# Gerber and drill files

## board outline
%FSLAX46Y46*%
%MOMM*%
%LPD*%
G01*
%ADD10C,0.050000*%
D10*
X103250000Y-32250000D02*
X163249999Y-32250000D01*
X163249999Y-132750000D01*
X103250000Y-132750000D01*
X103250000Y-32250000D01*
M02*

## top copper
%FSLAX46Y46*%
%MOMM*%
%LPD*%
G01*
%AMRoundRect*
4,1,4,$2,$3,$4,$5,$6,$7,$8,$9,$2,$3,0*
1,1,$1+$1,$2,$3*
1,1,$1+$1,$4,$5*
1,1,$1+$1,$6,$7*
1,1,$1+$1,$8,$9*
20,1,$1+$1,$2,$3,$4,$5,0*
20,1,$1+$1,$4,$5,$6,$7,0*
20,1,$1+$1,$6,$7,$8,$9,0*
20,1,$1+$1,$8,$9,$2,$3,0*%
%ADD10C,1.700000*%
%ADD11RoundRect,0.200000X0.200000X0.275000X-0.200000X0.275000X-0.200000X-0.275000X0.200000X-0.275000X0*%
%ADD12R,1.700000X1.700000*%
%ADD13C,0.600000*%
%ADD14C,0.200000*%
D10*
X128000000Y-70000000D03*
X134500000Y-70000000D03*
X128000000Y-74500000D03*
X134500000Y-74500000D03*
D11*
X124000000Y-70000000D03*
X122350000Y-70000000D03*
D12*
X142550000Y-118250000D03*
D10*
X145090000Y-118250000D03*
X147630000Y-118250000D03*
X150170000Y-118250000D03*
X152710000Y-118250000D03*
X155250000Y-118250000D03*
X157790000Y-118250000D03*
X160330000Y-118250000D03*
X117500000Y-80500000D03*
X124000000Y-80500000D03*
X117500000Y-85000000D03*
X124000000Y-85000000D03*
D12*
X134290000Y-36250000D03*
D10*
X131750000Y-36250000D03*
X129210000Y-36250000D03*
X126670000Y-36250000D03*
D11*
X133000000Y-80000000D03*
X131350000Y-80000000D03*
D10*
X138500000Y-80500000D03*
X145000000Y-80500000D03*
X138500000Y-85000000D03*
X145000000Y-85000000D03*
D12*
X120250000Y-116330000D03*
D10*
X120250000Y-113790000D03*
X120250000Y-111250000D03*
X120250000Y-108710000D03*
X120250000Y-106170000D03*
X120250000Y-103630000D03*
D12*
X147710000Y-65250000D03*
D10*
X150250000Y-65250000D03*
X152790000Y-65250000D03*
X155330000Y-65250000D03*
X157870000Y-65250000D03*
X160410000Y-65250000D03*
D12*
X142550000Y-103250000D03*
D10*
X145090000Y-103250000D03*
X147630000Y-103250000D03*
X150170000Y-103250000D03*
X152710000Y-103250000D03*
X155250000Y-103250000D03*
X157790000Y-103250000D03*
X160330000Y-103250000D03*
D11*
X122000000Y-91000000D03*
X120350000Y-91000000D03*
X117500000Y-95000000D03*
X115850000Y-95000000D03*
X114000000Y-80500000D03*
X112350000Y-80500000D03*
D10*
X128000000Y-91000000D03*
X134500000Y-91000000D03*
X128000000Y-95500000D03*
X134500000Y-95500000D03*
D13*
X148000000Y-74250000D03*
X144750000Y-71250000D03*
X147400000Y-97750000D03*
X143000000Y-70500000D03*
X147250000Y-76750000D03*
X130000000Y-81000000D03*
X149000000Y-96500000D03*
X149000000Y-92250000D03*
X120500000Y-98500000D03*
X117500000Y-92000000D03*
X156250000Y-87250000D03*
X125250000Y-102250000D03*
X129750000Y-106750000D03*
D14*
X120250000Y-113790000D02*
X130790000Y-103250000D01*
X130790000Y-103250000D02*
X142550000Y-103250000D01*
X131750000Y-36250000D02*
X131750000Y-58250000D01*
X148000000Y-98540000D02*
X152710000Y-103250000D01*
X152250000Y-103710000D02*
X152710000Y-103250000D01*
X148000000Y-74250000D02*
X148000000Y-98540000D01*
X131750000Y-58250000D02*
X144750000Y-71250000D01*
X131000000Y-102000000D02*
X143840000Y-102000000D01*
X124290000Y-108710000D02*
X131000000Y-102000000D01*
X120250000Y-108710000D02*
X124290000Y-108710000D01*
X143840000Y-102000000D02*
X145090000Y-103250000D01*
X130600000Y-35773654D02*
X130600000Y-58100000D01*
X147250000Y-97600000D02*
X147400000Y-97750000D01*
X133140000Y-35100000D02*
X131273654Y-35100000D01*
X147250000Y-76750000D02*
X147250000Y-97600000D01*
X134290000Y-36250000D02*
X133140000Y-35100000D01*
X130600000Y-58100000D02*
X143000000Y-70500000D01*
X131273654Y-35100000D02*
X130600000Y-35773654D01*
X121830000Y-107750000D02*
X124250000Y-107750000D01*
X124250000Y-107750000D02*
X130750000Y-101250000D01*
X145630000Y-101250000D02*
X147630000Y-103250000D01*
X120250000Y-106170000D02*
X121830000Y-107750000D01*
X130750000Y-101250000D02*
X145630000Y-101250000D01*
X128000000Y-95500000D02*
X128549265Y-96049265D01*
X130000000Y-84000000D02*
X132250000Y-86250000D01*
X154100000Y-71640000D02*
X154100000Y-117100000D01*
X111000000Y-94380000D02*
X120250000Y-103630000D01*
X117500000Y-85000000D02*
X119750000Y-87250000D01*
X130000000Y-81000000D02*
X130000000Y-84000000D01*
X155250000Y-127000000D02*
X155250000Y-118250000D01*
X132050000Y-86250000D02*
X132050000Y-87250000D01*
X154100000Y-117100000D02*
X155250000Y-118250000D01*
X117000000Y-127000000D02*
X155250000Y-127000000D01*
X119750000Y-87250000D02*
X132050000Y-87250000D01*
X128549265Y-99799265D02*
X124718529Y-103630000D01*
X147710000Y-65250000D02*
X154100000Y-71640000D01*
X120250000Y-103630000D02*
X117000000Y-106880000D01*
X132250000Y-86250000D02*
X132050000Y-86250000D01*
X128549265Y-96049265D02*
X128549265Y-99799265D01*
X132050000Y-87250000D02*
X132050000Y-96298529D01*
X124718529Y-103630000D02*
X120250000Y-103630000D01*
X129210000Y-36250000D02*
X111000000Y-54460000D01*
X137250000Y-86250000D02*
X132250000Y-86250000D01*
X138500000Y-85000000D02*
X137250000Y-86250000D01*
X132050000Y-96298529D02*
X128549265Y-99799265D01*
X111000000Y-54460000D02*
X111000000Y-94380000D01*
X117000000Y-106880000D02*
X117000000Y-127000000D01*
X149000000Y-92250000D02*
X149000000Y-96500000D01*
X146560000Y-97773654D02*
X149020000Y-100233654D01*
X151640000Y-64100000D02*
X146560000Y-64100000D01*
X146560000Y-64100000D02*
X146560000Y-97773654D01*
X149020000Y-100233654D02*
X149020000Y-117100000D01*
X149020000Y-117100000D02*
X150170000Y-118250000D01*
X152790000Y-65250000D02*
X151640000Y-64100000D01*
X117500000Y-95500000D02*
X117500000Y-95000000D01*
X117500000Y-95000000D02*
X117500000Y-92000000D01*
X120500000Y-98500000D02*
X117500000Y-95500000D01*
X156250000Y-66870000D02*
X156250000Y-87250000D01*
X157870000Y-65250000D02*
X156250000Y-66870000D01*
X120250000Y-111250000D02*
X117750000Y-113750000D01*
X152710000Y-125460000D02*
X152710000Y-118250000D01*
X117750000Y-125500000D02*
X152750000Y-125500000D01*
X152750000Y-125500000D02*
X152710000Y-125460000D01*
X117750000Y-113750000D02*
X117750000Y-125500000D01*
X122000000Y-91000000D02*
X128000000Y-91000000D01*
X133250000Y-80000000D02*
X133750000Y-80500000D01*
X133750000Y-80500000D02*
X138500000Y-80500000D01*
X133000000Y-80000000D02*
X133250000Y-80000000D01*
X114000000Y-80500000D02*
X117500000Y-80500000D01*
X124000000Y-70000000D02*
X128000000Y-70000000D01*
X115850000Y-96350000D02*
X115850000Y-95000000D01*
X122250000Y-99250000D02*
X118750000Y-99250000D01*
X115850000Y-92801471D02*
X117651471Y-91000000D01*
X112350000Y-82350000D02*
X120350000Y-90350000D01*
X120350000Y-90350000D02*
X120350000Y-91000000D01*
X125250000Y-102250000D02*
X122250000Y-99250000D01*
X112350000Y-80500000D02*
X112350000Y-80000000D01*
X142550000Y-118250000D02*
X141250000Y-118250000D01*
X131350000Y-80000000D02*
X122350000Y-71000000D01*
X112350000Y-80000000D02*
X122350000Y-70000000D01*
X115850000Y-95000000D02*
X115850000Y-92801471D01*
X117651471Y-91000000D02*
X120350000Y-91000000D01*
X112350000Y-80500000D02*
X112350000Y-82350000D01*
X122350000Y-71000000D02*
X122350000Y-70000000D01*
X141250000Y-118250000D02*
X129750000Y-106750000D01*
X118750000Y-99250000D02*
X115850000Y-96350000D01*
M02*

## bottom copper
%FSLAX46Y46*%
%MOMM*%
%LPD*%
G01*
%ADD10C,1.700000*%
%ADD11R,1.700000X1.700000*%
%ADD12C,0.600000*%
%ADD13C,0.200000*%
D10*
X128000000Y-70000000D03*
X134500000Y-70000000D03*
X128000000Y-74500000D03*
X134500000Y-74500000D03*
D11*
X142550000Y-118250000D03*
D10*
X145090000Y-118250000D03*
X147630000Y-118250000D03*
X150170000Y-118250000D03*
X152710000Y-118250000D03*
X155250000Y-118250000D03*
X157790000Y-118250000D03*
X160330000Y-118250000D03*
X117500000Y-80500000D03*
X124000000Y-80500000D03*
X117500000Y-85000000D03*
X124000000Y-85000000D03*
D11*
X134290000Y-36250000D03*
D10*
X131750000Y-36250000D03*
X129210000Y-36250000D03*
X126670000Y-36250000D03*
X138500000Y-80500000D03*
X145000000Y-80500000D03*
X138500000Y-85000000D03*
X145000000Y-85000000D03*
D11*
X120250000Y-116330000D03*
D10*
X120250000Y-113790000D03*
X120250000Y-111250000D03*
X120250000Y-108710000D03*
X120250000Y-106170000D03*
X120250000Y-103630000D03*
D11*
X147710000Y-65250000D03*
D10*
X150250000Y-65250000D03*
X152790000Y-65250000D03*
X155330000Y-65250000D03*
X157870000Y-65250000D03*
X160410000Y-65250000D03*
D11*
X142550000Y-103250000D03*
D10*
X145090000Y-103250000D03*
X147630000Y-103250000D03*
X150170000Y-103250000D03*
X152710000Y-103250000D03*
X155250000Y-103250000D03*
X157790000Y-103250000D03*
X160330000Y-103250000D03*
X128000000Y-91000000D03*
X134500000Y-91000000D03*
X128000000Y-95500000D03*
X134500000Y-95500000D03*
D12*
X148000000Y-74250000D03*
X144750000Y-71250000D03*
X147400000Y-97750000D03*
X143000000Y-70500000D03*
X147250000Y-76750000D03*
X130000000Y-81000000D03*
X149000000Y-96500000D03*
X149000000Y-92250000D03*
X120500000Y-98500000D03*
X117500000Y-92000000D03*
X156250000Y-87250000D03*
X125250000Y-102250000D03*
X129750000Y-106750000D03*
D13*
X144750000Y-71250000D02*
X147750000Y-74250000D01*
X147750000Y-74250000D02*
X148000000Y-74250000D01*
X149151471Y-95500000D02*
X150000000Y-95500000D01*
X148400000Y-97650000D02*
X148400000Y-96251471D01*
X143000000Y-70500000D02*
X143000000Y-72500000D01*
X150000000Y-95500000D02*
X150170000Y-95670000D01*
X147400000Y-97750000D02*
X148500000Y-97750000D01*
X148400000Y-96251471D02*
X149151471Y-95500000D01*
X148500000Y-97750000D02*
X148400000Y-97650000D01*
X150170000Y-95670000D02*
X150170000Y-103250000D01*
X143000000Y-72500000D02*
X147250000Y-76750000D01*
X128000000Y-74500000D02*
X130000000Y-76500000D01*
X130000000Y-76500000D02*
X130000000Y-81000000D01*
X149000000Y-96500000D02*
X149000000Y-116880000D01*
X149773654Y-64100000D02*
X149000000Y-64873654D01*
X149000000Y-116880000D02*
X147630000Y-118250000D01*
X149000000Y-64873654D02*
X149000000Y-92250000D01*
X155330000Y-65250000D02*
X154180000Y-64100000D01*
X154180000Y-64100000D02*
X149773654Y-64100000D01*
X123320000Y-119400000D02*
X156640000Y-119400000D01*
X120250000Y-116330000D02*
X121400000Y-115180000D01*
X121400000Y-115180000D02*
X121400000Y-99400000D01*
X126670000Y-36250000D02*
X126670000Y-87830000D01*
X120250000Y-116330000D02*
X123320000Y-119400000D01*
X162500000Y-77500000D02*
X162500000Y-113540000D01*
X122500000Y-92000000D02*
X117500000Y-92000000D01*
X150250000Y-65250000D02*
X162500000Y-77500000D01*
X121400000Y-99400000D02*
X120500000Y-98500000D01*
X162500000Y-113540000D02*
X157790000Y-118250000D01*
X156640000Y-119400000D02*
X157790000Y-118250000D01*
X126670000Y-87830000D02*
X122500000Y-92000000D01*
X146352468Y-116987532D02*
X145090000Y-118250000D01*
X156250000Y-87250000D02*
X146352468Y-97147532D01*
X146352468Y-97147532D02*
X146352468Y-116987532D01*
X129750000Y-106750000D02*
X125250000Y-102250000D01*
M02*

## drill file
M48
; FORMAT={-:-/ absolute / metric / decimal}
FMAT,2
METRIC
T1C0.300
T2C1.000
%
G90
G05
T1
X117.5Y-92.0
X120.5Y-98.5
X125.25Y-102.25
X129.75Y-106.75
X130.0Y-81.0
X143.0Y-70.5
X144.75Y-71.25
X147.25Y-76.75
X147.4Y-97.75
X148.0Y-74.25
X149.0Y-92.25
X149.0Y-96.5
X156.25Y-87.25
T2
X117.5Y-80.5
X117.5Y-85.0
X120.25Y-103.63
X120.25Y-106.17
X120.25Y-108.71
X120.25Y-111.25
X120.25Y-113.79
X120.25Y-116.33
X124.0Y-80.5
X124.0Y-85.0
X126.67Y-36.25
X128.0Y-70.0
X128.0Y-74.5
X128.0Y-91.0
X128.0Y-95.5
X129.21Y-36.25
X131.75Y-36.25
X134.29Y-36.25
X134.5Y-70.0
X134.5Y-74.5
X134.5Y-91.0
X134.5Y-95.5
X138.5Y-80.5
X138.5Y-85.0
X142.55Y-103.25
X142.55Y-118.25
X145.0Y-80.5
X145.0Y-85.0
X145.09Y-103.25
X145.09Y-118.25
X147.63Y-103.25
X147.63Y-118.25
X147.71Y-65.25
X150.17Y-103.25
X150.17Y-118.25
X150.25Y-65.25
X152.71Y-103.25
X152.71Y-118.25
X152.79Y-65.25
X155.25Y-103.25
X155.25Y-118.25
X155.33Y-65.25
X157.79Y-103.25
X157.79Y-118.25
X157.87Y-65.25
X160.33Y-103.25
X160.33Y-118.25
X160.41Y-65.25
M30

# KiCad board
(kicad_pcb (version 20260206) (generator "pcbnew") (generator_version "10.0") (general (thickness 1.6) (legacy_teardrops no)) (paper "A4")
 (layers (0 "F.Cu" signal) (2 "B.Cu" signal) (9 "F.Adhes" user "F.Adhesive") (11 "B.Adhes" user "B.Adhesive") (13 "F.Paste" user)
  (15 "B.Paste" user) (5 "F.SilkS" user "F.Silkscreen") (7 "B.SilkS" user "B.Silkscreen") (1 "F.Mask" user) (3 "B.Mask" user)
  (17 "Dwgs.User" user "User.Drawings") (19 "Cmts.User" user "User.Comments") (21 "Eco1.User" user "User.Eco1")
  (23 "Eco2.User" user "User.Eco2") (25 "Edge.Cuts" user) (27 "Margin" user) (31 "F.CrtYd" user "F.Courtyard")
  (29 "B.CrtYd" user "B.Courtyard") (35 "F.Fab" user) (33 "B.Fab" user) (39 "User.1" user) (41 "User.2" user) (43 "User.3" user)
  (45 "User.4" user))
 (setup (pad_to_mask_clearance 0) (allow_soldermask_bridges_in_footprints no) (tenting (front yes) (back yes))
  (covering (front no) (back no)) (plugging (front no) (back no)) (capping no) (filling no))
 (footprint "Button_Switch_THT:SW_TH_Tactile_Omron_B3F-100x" (layer "F.Cu") (at 128 70)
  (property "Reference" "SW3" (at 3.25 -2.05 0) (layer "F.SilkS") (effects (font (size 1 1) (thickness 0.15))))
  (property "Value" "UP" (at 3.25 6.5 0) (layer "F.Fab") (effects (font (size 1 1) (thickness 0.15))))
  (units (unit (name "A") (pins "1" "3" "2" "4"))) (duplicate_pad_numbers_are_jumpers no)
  (pad "1" thru_hole circle (at 0 0) (size 1.7 1.7) (drill 1) (layers "*.Cu" "*.Mask") (remove_unused_layers no) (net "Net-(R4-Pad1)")
   (thermal_bridge_angle 90))
  (pad "1" thru_hole circle (at 6.5 0) (size 1.7 1.7) (drill 1) (layers "*.Cu" "*.Mask") (remove_unused_layers no) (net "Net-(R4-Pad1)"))
  (pad "2" thru_hole circle (at 0 4.5) (size 1.7 1.7) (drill 1) (layers "*.Cu" "*.Mask") (remove_unused_layers no) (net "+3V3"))
  (pad "2" thru_hole circle (at 6.5 4.5) (size 1.7 1.7) (drill 1) (layers "*.Cu" "*.Mask") (remove_unused_layers no)
   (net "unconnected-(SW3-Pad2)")))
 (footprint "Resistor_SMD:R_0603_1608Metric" (layer "F.Cu") (at 123.175 70 180)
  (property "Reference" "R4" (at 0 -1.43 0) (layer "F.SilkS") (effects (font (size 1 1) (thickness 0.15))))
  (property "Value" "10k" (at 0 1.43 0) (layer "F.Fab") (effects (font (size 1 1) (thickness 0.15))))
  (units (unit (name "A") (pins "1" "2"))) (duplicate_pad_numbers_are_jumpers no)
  (pad "1" smd roundrect (at -0.825 0 180) (size 0.8 0.95) (layers "F.Cu" "F.Mask" "F.Paste") (roundrect_rratio 0.25) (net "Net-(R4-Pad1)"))
  (pad "2" smd roundrect (at 0.825 0 180) (size 0.8 0.95) (layers "F.Cu" "F.Mask" "F.Paste") (roundrect_rratio 0.25) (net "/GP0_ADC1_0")))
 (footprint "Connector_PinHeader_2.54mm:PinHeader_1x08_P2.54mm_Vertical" (layer "F.Cu") (at 142.55 118.25 90)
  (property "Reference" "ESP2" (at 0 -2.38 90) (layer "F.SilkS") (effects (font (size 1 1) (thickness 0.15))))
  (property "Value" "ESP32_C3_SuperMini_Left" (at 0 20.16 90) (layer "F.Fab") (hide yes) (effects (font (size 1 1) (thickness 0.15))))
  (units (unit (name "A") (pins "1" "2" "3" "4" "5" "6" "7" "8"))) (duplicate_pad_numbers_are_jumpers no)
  (pad "1" thru_hole rect (at 0 0 90) (size 1.7 1.7) (drill 1) (layers "*.Cu" "*.Mask") (remove_unused_layers no) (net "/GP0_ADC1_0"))
  (pad "2" thru_hole circle (at 0 2.54 90) (size 1.7 1.7) (drill 1) (layers "*.Cu" "*.Mask") (remove_unused_layers no) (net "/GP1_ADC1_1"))
  (pad "3" thru_hole circle (at 0 5.08 90) (size 1.7 1.7) (drill 1) (layers "*.Cu" "*.Mask") (remove_unused_layers no) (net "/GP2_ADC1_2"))
  (pad "4" thru_hole circle (at 0 7.62 90) (size 1.7 1.7) (drill 1) (layers "*.Cu" "*.Mask") (remove_unused_layers no) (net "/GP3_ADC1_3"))
  (pad "5" thru_hole circle (at 0 10.16 90) (size 1.7 1.7) (drill 1) (layers "*.Cu" "*.Mask") (remove_unused_layers no) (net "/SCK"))
  (pad "6" thru_hole circle (at 0 12.7 90) (size 1.7 1.7) (drill 1) (layers "*.Cu" "*.Mask") (remove_unused_layers no) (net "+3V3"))
  (pad "7" thru_hole circle (at 0 15.24 90) (size 1.7 1.7) (drill 1) (layers "*.Cu" "*.Mask") (remove_unused_layers no) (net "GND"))
  (pad "8" thru_hole circle (at 0 17.78 90) (size 1.7 1.7) (drill 1) (layers "*.Cu" "*.Mask") (remove_unused_layers no)
   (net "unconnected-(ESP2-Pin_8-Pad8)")))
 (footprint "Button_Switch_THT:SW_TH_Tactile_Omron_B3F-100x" (layer "F.Cu") (at 117.5 80.5)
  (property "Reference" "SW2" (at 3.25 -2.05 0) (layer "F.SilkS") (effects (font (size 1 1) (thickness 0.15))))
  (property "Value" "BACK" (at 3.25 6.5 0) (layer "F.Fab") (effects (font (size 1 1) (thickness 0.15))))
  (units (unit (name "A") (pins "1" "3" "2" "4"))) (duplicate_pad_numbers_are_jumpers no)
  (pad "1" thru_hole circle (at 0 0) (size 1.7 1.7) (drill 1) (layers "*.Cu" "*.Mask") (remove_unused_layers no) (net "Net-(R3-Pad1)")
   (thermal_bridge_angle 90))
  (pad "1" thru_hole circle (at 6.5 0) (size 1.7 1.7) (drill 1) (layers "*.Cu" "*.Mask") (remove_unused_layers no) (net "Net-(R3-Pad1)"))
  (pad "2" thru_hole circle (at 0 4.5) (size 1.7 1.7) (drill 1) (layers "*.Cu" "*.Mask") (remove_unused_layers no) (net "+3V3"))
  (pad "2" thru_hole circle (at 6.5 4.5) (size 1.7 1.7) (drill 1) (layers "*.Cu" "*.Mask") (remove_unused_layers no)
   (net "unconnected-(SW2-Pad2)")))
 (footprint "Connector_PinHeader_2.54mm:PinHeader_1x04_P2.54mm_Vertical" (layer "F.Cu") (at 134.29 36.25 -90)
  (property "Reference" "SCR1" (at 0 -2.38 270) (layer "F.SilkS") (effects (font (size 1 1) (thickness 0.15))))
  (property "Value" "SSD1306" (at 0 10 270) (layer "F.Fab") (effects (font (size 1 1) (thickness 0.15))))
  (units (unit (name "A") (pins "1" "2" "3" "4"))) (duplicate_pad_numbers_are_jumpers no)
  (pad "1" thru_hole rect (at 0 0 270) (size 1.7 1.7) (drill 1) (layers "*.Cu" "*.Mask") (remove_unused_layers no) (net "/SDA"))
  (pad "2" thru_hole circle (at 0 2.54 270) (size 1.7 1.7) (drill 1) (layers "*.Cu" "*.Mask") (remove_unused_layers no) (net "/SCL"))
  (pad "3" thru_hole circle (at 0 5.08 270) (size 1.7 1.7) (drill 1) (layers "*.Cu" "*.Mask") (remove_unused_layers no) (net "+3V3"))
  (pad "4" thru_hole circle (at 0 7.62 270) (size 1.7 1.7) (drill 1) (layers "*.Cu" "*.Mask") (remove_unused_layers no) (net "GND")))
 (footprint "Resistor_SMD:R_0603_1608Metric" (layer "F.Cu") (at 132.175 80 180)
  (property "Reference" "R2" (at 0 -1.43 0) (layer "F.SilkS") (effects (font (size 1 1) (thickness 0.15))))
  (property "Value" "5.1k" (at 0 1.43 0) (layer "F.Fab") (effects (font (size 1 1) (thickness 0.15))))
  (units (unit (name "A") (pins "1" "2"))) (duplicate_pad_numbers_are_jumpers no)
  (pad "1" smd roundrect (at -0.825 0 180) (size 0.8 0.95) (layers "F.Cu" "F.Mask" "F.Paste") (roundrect_rratio 0.25) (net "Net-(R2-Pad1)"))
  (pad "2" smd roundrect (at 0.825 0 180) (size 0.8 0.95) (layers "F.Cu" "F.Mask" "F.Paste") (roundrect_rratio 0.25) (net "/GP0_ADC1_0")))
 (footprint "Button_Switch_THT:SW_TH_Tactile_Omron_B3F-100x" (layer "F.Cu") (at 138.5 80.5)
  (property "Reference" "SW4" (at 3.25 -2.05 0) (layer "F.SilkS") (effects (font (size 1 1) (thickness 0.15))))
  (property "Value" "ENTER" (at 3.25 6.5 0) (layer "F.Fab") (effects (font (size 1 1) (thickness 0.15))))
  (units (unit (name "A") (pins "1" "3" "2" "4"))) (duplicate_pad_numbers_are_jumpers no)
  (pad "1" thru_hole circle (at 0 0) (size 1.7 1.7) (drill 1) (layers "*.Cu" "*.Mask") (remove_unused_layers no) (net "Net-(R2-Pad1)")
   (thermal_bridge_angle 90))
  (pad "1" thru_hole circle (at 6.5 0) (size 1.7 1.7) (drill 1) (layers "*.Cu" "*.Mask") (remove_unused_layers no) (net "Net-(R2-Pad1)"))
  (pad "2" thru_hole circle (at 0 4.5) (size 1.7 1.7) (drill 1) (layers "*.Cu" "*.Mask") (remove_unused_layers no) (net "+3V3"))
  (pad "2" thru_hole circle (at 6.5 4.5) (size 1.7 1.7) (drill 1) (layers "*.Cu" "*.Mask") (remove_unused_layers no)
   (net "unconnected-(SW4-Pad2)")))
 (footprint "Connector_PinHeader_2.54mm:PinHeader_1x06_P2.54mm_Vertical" (layer "F.Cu") (at 120.25 116.33 180)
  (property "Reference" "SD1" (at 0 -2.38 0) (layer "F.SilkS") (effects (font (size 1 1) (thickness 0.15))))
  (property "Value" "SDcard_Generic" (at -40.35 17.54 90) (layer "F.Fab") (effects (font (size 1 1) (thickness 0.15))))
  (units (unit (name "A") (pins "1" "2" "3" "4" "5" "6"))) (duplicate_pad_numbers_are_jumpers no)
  (pad "1" thru_hole rect (at 0 0 180) (size 1.7 1.7) (drill 1) (layers "*.Cu" "*.Mask") (remove_unused_layers no) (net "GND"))
  (pad "2" thru_hole circle (at 0 2.54 180) (size 1.7 1.7) (drill 1) (layers "*.Cu" "*.Mask") (remove_unused_layers no) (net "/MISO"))
  (pad "3" thru_hole circle (at 0 5.08 180) (size 1.7 1.7) (drill 1) (layers "*.Cu" "*.Mask") (remove_unused_layers no) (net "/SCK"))
  (pad "4" thru_hole circle (at 0 7.62 180) (size 1.7 1.7) (drill 1) (layers "*.Cu" "*.Mask") (remove_unused_layers no) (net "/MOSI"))
  (pad "5" thru_hole circle (at 0 10.16 180) (size 1.7 1.7) (drill 1) (layers "*.Cu" "*.Mask") (remove_unused_layers no) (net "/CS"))
  (pad "6" thru_hole circle (at 0 12.7 180) (size 1.7 1.7) (drill 1) (layers "*.Cu" "*.Mask") (remove_unused_layers no) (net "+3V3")))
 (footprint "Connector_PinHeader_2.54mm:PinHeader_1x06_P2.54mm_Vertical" (layer "F.Cu") (at 147.71 65.25 90)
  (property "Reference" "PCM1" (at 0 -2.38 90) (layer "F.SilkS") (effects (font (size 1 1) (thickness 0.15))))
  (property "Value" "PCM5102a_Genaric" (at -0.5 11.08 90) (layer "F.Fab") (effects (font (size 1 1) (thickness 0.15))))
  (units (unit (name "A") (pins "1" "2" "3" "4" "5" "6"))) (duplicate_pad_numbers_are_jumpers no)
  (pad "1" thru_hole rect (at 0 0 90) (size 1.7 1.7) (drill 1) (layers "*.Cu" "*.Mask") (remove_unused_layers no) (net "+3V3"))
  (pad "2" thru_hole circle (at 0 2.54 90) (size 1.7 1.7) (drill 1) (layers "*.Cu" "*.Mask") (remove_unused_layers no) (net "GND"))
  (pad "3" thru_hole circle (at 0 5.08 90) (size 1.7 1.7) (drill 1) (layers "*.Cu" "*.Mask") (remove_unused_layers no) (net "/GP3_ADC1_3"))
  (pad "4" thru_hole circle (at 0 7.62 90) (size 1.7 1.7) (drill 1) (layers "*.Cu" "*.Mask") (remove_unused_layers no) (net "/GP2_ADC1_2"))
  (pad "5" thru_hole circle (at 0 10.16 90) (size 1.7 1.7) (drill 1) (layers "*.Cu" "*.Mask") (remove_unused_layers no) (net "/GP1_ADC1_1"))
  (pad "6" thru_hole circle (at 0 12.7 90) (size 1.7 1.7) (drill 1) (layers "*.Cu" "*.Mask") (remove_unused_layers no)
   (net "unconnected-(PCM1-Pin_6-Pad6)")))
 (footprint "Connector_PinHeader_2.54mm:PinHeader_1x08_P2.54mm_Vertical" (layer "F.Cu") (at 142.55 103.25 90)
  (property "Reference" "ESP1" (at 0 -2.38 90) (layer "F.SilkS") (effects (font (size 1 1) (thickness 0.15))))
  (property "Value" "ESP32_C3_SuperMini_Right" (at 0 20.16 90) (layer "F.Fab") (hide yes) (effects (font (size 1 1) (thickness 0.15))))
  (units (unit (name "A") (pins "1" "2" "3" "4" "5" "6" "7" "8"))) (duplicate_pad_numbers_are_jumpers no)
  (pad "1" thru_hole rect (at 0 0 90) (size 1.7 1.7) (drill 1) (layers "*.Cu" "*.Mask") (remove_unused_layers no) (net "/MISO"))
  (pad "2" thru_hole circle (at 0 2.54 90) (size 1.7 1.7) (drill 1) (layers "*.Cu" "*.Mask") (remove_unused_layers no) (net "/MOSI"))
  (pad "3" thru_hole circle (at 0 5.08 90) (size 1.7 1.7) (drill 1) (layers "*.Cu" "*.Mask") (remove_unused_layers no) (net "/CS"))
  (pad "4" thru_hole circle (at 0 7.62 90) (size 1.7 1.7) (drill 1) (layers "*.Cu" "*.Mask") (remove_unused_layers no) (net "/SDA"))
  (pad "5" thru_hole circle (at 0 10.16 90) (size 1.7 1.7) (drill 1) (layers "*.Cu" "*.Mask") (remove_unused_layers no) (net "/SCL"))
  (pad "6" thru_hole circle (at 0 12.7 90) (size 1.7 1.7) (drill 1) (layers "*.Cu" "*.Mask") (remove_unused_layers no)
   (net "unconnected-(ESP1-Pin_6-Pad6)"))
  (pad "7" thru_hole circle (at 0 15.24 90) (size 1.7 1.7) (drill 1) (layers "*.Cu" "*.Mask") (remove_unused_layers no)
   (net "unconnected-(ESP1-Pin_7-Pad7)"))
  (pad "8" thru_hole circle (at 0 17.78 90) (size 1.7 1.7) (drill 1) (layers "*.Cu" "*.Mask") (remove_unused_layers no)
   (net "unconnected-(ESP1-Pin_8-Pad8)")))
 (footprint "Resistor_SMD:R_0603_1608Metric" (layer "F.Cu") (at 121.175 91 180)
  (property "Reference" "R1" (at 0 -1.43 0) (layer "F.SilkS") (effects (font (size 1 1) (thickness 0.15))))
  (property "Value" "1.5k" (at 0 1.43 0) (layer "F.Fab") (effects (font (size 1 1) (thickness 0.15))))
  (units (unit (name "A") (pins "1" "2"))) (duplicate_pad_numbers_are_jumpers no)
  (pad "1" smd roundrect (at -0.825 0 180) (size 0.8 0.95) (layers "F.Cu" "F.Mask" "F.Paste") (roundrect_rratio 0.25) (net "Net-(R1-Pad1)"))
  (pad "2" smd roundrect (at 0.825 0 180) (size 0.8 0.95) (layers "F.Cu" "F.Mask" "F.Paste") (roundrect_rratio 0.25) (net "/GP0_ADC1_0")))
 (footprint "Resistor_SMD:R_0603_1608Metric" (layer "F.Cu") (at 116.675 95 180)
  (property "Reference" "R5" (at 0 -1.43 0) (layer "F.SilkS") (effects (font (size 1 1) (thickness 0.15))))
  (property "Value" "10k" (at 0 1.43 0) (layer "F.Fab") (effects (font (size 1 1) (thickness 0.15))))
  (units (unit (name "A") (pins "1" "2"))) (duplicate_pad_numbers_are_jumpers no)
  (pad "1" smd roundrect (at -0.825 0 180) (size 0.8 0.95) (layers "F.Cu" "F.Mask" "F.Paste") (roundrect_rratio 0.25) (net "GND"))
  (pad "2" smd roundrect (at 0.825 0 180) (size 0.8 0.95) (layers "F.Cu" "F.Mask" "F.Paste") (roundrect_rratio 0.25) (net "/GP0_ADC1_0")))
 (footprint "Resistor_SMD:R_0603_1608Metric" (layer "F.Cu") (at 113.175 80.5 180)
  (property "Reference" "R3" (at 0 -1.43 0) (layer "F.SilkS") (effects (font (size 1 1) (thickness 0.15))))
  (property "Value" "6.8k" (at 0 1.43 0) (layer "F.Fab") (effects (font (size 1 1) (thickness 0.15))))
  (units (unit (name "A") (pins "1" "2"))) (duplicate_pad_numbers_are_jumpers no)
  (pad "1" smd roundrect (at -0.825 0 180) (size 0.8 0.95) (layers "F.Cu" "F.Mask" "F.Paste") (roundrect_rratio 0.25) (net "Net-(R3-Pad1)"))
  (pad "2" smd roundrect (at 0.825 0 180) (size 0.8 0.95) (layers "F.Cu" "F.Mask" "F.Paste") (roundrect_rratio 0.25) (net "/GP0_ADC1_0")))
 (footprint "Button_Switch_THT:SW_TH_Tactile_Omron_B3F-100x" (layer "F.Cu") (at 128 91)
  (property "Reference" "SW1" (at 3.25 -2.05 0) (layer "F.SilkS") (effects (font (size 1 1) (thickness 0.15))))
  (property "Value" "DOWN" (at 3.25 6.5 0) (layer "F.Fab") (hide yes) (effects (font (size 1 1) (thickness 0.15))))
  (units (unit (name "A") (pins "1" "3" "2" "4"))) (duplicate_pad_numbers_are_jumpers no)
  (pad "1" thru_hole circle (at 0 0) (size 1.7 1.7) (drill 1) (layers "*.Cu" "*.Mask") (remove_unused_layers no) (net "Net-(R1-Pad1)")
   (thermal_bridge_angle 90))
  (pad "1" thru_hole circle (at 6.5 0) (size 1.7 1.7) (drill 1) (layers "*.Cu" "*.Mask") (remove_unused_layers no) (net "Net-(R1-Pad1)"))
  (pad "2" thru_hole circle (at 0 4.5) (size 1.7 1.7) (drill 1) (layers "*.Cu" "*.Mask") (remove_unused_layers no) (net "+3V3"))
  (pad "2" thru_hole circle (at 6.5 4.5) (size 1.7 1.7) (drill 1) (layers "*.Cu" "*.Mask") (remove_unused_layers no)
   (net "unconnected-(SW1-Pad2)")))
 (gr_rect (start 103.25 32.25) (end 163.249999 132.75) (stroke (width 0.05) (type default)) (fill no) (layer "Edge.Cuts"))
 (segment (start 120.25 113.79) (end 130.79 103.25) (width 0.2) (layer "F.Cu") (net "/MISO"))
 (segment (start 130.79 103.25) (end 142.55 103.25) (width 0.2) (layer "F.Cu") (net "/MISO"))
 (segment (start 131.75 36.25) (end 131.75 58.25) (width 0.2) (layer "F.Cu") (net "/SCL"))
 (segment (start 148 98.54) (end 152.71 103.25) (width 0.2) (layer "F.Cu") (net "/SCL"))
 (segment (start 152.25 103.71) (end 152.71 103.25) (width 0.2) (layer "F.Cu") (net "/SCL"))
 (segment (start 148 74.25) (end 148 98.54) (width 0.2) (layer "F.Cu") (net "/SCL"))
 (segment (start 131.75 58.25) (end 144.75 71.25) (width 0.2) (layer "F.Cu") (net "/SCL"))
 (via (at 148 74.25) (size 0.6) (drill 0.3) (layers "F.Cu" "B.Cu") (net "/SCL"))
 (via (at 144.75 71.25) (size 0.6) (drill 0.3) (layers "F.Cu" "B.Cu") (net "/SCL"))
 (segment (start 144.75 71.25) (end 147.75 74.25) (width 0.2) (layer "B.Cu") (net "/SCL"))
 (segment (start 147.75 74.25) (end 148 74.25) (width 0.2) (layer "B.Cu") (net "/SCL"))
 (segment (start 131 102) (end 143.84 102) (width 0.2) (layer "F.Cu") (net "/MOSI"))
 (segment (start 124.29 108.71) (end 131 102) (width 0.2) (layer "F.Cu") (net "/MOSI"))
 (segment (start 120.25 108.71) (end 124.29 108.71) (width 0.2) (layer "F.Cu") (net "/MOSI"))
 (segment (start 143.84 102) (end 145.09 103.25) (width 0.2) (layer "F.Cu") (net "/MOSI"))
 (segment (start 130.6 35.773654) (end 130.6 58.1) (width 0.2) (layer "F.Cu") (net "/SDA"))
 (segment (start 147.25 97.6) (end 147.4 97.75) (width 0.2) (layer "F.Cu") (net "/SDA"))
 (segment (start 133.14 35.1) (end 131.273654 35.1) (width 0.2) (layer "F.Cu") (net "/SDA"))
 (segment (start 147.25 76.75) (end 147.25 97.6) (width 0.2) (layer "F.Cu") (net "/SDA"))
 (segment (start 134.29 36.25) (end 133.14 35.1) (width 0.2) (layer "F.Cu") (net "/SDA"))
 (segment (start 130.6 58.1) (end 143 70.5) (width 0.2) (layer "F.Cu") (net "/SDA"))
 (segment (start 131.273654 35.1) (end 130.6 35.773654) (width 0.2) (layer "F.Cu") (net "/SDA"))
 (via (at 147.4 97.75) (size 0.6) (drill 0.3) (layers "F.Cu" "B.Cu") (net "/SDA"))
 (via (at 143 70.5) (size 0.6) (drill 0.3) (layers "F.Cu" "B.Cu") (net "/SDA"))
 (via (at 147.25 76.75) (size 0.6) (drill 0.3) (layers "F.Cu" "B.Cu") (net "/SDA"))
 (segment (start 149.151471 95.5) (end 150 95.5) (width 0.2) (layer "B.Cu") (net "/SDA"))
 (segment (start 148.4 97.65) (end 148.4 96.251471) (width 0.2) (layer "B.Cu") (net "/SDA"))
 (segment (start 143 70.5) (end 143 72.5) (width 0.2) (layer "B.Cu") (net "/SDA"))
 (segment (start 150 95.5) (end 150.17 95.67) (width 0.2) (layer "B.Cu") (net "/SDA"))
 (segment (start 147.4 97.75) (end 148.5 97.75) (width 0.2) (layer "B.Cu") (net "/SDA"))
 (segment (start 148.4 96.251471) (end 149.151471 95.5) (width 0.2) (layer "B.Cu") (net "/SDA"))
 (segment (start 148.5 97.75) (end 148.4 97.65) (width 0.2) (layer "B.Cu") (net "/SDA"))
 (segment (start 150.17 95.67) (end 150.17 103.25) (width 0.2) (layer "B.Cu") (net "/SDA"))
 (segment (start 143 72.5) (end 147.25 76.75) (width 0.2) (layer "B.Cu") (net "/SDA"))
 (segment (start 121.83 107.75) (end 124.25 107.75) (width 0.2) (layer "F.Cu") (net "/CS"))
 (segment (start 124.25 107.75) (end 130.75 101.25) (width 0.2) (layer "F.Cu") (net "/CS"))
 (segment (start 145.63 101.25) (end 147.63 103.25) (width 0.2) (layer "F.Cu") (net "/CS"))
 (segment (start 120.25 106.17) (end 121.83 107.75) (width 0.2) (layer "F.Cu") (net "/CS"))
 (segment (start 130.75 101.25) (end 145.63 101.25) (width 0.2) (layer "F.Cu") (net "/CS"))
 (segment (start 128 95.5) (end 128.549265 96.049265) (width 0.2) (layer "F.Cu") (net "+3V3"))
 (segment (start 130 84) (end 132.25 86.25) (width 0.2) (layer "F.Cu") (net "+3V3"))
 (segment (start 154.1 71.64) (end 154.1 117.1) (width 0.2) (layer "F.Cu") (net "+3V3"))
 (segment (start 111 94.38) (end 120.25 103.63) (width 0.2) (layer "F.Cu") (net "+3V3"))
 (segment (start 117.5 85) (end 119.75 87.25) (width 0.2) (layer "F.Cu") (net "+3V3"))
 (segment (start 130 81) (end 130 84) (width 0.2) (layer "F.Cu") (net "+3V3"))
 (segment (start 155.25 127) (end 155.25 118.25) (width 0.2) (layer "F.Cu") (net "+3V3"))
 (segment (start 132.05 86.25) (end 132.05 87.25) (width 0.2) (layer "F.Cu") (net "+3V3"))
 (segment (start 154.1 117.1) (end 155.25 118.25) (width 0.2) (layer "F.Cu") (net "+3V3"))
 (segment (start 117 127) (end 155.25 127) (width 0.2) (layer "F.Cu") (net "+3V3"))
 (segment (start 119.75 87.25) (end 132.05 87.25) (width 0.2) (layer "F.Cu") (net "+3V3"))
 (segment (start 128.549265 99.799265) (end 124.718529 103.63) (width 0.2) (layer "F.Cu") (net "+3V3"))
 (segment (start 147.71 65.25) (end 154.1 71.64) (width 0.2) (layer "F.Cu") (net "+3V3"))
 (segment (start 120.25 103.63) (end 117 106.88) (width 0.2) (layer "F.Cu") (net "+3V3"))
 (segment (start 132.25 86.25) (end 132.05 86.25) (width 0.2) (layer "F.Cu") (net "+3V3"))
 (segment (start 128.549265 96.049265) (end 128.549265 99.799265) (width 0.2) (layer "F.Cu") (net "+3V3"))
 (segment (start 132.05 87.25) (end 132.05 96.298529) (width 0.2) (layer "F.Cu") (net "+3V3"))
 (segment (start 124.718529 103.63) (end 120.25 103.63) (width 0.2) (layer "F.Cu") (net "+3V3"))
 (segment (start 129.21 36.25) (end 111 54.46) (width 0.2) (layer "F.Cu") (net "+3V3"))
 (segment (start 137.25 86.25) (end 132.25 86.25) (width 0.2) (layer "F.Cu") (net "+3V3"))
 (segment (start 138.5 85) (end 137.25 86.25) (width 0.2) (layer "F.Cu") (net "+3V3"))
 (segment (start 132.05 96.298529) (end 128.549265 99.799265) (width 0.2) (layer "F.Cu") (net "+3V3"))
 (segment (start 111 54.46) (end 111 94.38) (width 0.2) (layer "F.Cu") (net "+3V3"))
 (segment (start 117 106.88) (end 117 127) (width 0.2) (layer "F.Cu") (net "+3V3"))
 (via (at 130 81) (size 0.6) (drill 0.3) (layers "F.Cu" "B.Cu") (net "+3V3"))
 (segment (start 128 74.5) (end 130 76.5) (width 0.2) (layer "B.Cu") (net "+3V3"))
 (segment (start 130 76.5) (end 130 81) (width 0.2) (layer "B.Cu") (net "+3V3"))
 (segment (start 149 92.25) (end 149 96.5) (width 0.2) (layer "F.Cu") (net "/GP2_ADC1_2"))
 (via (at 149 96.5) (size 0.6) (drill 0.3) (layers "F.Cu" "B.Cu") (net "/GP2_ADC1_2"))
 (via (at 149 92.25) (size 0.6) (drill 0.3) (layers "F.Cu" "B.Cu") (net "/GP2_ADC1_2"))
 (segment (start 149 96.5) (end 149 116.88) (width 0.2) (layer "B.Cu") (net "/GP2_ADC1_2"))
 (segment (start 149.773654 64.1) (end 149 64.873654) (width 0.2) (layer "B.Cu") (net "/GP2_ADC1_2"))
 (segment (start 149 116.88) (end 147.63 118.25) (width 0.2) (layer "B.Cu") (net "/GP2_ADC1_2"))
 (segment (start 149 64.873654) (end 149 92.25) (width 0.2) (layer "B.Cu") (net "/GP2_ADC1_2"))
 (segment (start 155.33 65.25) (end 154.18 64.1) (width 0.2) (layer "B.Cu") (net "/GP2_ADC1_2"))
 (segment (start 154.18 64.1) (end 149.773654 64.1) (width 0.2) (layer "B.Cu") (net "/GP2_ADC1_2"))
 (segment (start 146.56 97.773654) (end 149.02 100.233654) (width 0.2) (layer "F.Cu") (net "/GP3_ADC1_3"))
 (segment (start 151.64 64.1) (end 146.56 64.1) (width 0.2) (layer "F.Cu") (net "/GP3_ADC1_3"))
 (segment (start 146.56 64.1) (end 146.56 97.773654) (width 0.2) (layer "F.Cu") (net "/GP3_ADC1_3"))
 (segment (start 149.02 100.233654) (end 149.02 117.1) (width 0.2) (layer "F.Cu") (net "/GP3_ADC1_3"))
 (segment (start 149.02 117.1) (end 150.17 118.25) (width 0.2) (layer "F.Cu") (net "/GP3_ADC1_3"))
 (segment (start 152.79 65.25) (end 151.64 64.1) (width 0.2) (layer "F.Cu") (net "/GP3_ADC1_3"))
 (segment (start 117.5 95.5) (end 117.5 95) (width 0.2) (layer "F.Cu") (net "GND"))
 (segment (start 117.5 95) (end 117.5 92) (width 0.2) (layer "F.Cu") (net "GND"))
 (segment (start 120.5 98.5) (end 117.5 95.5) (width 0.2) (layer "F.Cu") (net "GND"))
 (via (at 120.5 98.5) (size 0.6) (drill 0.3) (layers "F.Cu" "B.Cu") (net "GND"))
 (via (at 117.5 92) (size 0.6) (drill 0.3) (layers "F.Cu" "B.Cu") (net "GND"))
 (segment (start 123.32 119.4) (end 156.64 119.4) (width 0.2) (layer "B.Cu") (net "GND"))
 (segment (start 120.25 116.33) (end 121.4 115.18) (width 0.2) (layer "B.Cu") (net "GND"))
 (segment (start 121.4 115.18) (end 121.4 99.4) (width 0.2) (layer "B.Cu") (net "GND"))
 (segment (start 126.67 36.25) (end 126.67 87.83) (width 0.2) (layer "B.Cu") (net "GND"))
 (segment (start 120.25 116.33) (end 123.32 119.4) (width 0.2) (layer "B.Cu") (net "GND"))
 (segment (start 162.5 77.5) (end 162.5 113.54) (width 0.2) (layer "B.Cu") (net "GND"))
 (segment (start 122.5 92) (end 117.5 92) (width 0.2) (layer "B.Cu") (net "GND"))
 (segment (start 150.25 65.25) (end 162.5 77.5) (width 0.2) (layer "B.Cu") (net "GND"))
 (segment (start 121.4 99.4) (end 120.5 98.5) (width 0.2) (layer "B.Cu") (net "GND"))
 (segment (start 162.5 113.54) (end 157.79 118.25) (width 0.2) (layer "B.Cu") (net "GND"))
 (segment (start 156.64 119.4) (end 157.79 118.25) (width 0.2) (layer "B.Cu") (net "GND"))
 (segment (start 126.67 87.83) (end 122.5 92) (width 0.2) (layer "B.Cu") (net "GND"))
 (segment (start 156.25 66.87) (end 156.25 87.25) (width 0.2) (layer "F.Cu") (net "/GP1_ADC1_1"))
 (segment (start 157.87 65.25) (end 156.25 66.87) (width 0.2) (layer "F.Cu") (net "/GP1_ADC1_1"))
 (via (at 156.25 87.25) (size 0.6) (drill 0.3) (layers "F.Cu" "B.Cu") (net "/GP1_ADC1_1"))
 (segment (start 146.352468 116.987532) (end 145.09 118.25) (width 0.2) (layer "B.Cu") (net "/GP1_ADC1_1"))
 (segment (start 156.25 87.25) (end 146.352468 97.147532) (width 0.2) (layer "B.Cu") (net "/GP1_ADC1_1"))
 (segment (start 146.352468 97.147532) (end 146.352468 116.987532) (width 0.2) (layer "B.Cu") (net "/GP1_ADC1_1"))
 (segment (start 120.25 111.25) (end 117.75 113.75) (width 0.2) (layer "F.Cu") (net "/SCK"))
 (segment (start 152.71 125.46) (end 152.71 118.25) (width 0.2) (layer "F.Cu") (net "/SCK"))
 (segment (start 117.75 125.5) (end 152.75 125.5) (width 0.2) (layer "F.Cu") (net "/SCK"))
 (segment (start 152.75 125.5) (end 152.71 125.46) (width 0.2) (layer "F.Cu") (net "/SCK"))
 (segment (start 117.75 113.75) (end 117.75 125.5) (width 0.2) (layer "F.Cu") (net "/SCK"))
 (segment (start 122 91) (end 128 91) (width 0.2) (layer "F.Cu") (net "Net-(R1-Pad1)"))
 (segment (start 133.25 80) (end 133.75 80.5) (width 0.2) (layer "F.Cu") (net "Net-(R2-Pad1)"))
 (segment (start 133.75 80.5) (end 138.5 80.5) (width 0.2) (layer "F.Cu") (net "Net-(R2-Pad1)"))
 (segment (start 133 80) (end 133.25 80) (width 0.2) (layer "F.Cu") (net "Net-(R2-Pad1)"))
 (segment (start 114 80.5) (end 117.5 80.5) (width 0.2) (layer "F.Cu") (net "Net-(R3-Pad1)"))
 (segment (start 124 70) (end 128 70) (width 0.2) (layer "F.Cu") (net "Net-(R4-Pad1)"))
 (segment (start 115.85 96.35) (end 115.85 95) (width 0.2) (layer "F.Cu") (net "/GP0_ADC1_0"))
 (segment (start 122.25 99.25) (end 118.75 99.25) (width 0.2) (layer "F.Cu") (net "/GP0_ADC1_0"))
 (segment (start 115.85 92.801471) (end 117.651471 91) (width 0.2) (layer "F.Cu") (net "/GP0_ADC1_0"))
 (segment (start 112.35 82.35) (end 120.35 90.35) (width 0.2) (layer "F.Cu") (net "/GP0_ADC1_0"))
 (segment (start 120.35 90.35) (end 120.35 91) (width 0.2) (layer "F.Cu") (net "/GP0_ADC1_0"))
 (segment (start 125.25 102.25) (end 122.25 99.25) (width 0.2) (layer "F.Cu") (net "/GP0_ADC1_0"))
 (segment (start 112.35 80.5) (end 112.35 80) (width 0.2) (layer "F.Cu") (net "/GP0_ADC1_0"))
 (segment (start 142.55 118.25) (end 141.25 118.25) (width 0.2) (layer "F.Cu") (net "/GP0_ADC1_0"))
 (segment (start 131.35 80) (end 122.35 71) (width 0.2) (layer "F.Cu") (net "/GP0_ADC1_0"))
 (segment (start 112.35 80) (end 122.35 70) (width 0.2) (layer "F.Cu") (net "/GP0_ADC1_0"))
 (segment (start 115.85 95) (end 115.85 92.801471) (width 0.2) (layer "F.Cu") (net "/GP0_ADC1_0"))
 (segment (start 117.651471 91) (end 120.35 91) (width 0.2) (layer "F.Cu") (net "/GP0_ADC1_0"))
 (segment (start 112.35 80.5) (end 112.35 82.35) (width 0.2) (layer "F.Cu") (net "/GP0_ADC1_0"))
 (segment (start 122.35 71) (end 122.35 70) (width 0.2) (layer "F.Cu") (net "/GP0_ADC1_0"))
 (segment (start 141.25 118.25) (end 129.75 106.75) (width 0.2) (layer "F.Cu") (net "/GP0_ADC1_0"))
 (segment (start 118.75 99.25) (end 115.85 96.35) (width 0.2) (layer "F.Cu") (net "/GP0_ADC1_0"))
 (via (at 125.25 102.25) (size 0.6) (drill 0.3) (layers "F.Cu" "B.Cu") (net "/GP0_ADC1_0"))
 (via (at 129.75 106.75) (size 0.6) (drill 0.3) (layers "F.Cu" "B.Cu") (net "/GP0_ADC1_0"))
 (segment (start 129.75 106.75) (end 125.25 102.25) (width 0.2) (layer "B.Cu") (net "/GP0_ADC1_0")))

